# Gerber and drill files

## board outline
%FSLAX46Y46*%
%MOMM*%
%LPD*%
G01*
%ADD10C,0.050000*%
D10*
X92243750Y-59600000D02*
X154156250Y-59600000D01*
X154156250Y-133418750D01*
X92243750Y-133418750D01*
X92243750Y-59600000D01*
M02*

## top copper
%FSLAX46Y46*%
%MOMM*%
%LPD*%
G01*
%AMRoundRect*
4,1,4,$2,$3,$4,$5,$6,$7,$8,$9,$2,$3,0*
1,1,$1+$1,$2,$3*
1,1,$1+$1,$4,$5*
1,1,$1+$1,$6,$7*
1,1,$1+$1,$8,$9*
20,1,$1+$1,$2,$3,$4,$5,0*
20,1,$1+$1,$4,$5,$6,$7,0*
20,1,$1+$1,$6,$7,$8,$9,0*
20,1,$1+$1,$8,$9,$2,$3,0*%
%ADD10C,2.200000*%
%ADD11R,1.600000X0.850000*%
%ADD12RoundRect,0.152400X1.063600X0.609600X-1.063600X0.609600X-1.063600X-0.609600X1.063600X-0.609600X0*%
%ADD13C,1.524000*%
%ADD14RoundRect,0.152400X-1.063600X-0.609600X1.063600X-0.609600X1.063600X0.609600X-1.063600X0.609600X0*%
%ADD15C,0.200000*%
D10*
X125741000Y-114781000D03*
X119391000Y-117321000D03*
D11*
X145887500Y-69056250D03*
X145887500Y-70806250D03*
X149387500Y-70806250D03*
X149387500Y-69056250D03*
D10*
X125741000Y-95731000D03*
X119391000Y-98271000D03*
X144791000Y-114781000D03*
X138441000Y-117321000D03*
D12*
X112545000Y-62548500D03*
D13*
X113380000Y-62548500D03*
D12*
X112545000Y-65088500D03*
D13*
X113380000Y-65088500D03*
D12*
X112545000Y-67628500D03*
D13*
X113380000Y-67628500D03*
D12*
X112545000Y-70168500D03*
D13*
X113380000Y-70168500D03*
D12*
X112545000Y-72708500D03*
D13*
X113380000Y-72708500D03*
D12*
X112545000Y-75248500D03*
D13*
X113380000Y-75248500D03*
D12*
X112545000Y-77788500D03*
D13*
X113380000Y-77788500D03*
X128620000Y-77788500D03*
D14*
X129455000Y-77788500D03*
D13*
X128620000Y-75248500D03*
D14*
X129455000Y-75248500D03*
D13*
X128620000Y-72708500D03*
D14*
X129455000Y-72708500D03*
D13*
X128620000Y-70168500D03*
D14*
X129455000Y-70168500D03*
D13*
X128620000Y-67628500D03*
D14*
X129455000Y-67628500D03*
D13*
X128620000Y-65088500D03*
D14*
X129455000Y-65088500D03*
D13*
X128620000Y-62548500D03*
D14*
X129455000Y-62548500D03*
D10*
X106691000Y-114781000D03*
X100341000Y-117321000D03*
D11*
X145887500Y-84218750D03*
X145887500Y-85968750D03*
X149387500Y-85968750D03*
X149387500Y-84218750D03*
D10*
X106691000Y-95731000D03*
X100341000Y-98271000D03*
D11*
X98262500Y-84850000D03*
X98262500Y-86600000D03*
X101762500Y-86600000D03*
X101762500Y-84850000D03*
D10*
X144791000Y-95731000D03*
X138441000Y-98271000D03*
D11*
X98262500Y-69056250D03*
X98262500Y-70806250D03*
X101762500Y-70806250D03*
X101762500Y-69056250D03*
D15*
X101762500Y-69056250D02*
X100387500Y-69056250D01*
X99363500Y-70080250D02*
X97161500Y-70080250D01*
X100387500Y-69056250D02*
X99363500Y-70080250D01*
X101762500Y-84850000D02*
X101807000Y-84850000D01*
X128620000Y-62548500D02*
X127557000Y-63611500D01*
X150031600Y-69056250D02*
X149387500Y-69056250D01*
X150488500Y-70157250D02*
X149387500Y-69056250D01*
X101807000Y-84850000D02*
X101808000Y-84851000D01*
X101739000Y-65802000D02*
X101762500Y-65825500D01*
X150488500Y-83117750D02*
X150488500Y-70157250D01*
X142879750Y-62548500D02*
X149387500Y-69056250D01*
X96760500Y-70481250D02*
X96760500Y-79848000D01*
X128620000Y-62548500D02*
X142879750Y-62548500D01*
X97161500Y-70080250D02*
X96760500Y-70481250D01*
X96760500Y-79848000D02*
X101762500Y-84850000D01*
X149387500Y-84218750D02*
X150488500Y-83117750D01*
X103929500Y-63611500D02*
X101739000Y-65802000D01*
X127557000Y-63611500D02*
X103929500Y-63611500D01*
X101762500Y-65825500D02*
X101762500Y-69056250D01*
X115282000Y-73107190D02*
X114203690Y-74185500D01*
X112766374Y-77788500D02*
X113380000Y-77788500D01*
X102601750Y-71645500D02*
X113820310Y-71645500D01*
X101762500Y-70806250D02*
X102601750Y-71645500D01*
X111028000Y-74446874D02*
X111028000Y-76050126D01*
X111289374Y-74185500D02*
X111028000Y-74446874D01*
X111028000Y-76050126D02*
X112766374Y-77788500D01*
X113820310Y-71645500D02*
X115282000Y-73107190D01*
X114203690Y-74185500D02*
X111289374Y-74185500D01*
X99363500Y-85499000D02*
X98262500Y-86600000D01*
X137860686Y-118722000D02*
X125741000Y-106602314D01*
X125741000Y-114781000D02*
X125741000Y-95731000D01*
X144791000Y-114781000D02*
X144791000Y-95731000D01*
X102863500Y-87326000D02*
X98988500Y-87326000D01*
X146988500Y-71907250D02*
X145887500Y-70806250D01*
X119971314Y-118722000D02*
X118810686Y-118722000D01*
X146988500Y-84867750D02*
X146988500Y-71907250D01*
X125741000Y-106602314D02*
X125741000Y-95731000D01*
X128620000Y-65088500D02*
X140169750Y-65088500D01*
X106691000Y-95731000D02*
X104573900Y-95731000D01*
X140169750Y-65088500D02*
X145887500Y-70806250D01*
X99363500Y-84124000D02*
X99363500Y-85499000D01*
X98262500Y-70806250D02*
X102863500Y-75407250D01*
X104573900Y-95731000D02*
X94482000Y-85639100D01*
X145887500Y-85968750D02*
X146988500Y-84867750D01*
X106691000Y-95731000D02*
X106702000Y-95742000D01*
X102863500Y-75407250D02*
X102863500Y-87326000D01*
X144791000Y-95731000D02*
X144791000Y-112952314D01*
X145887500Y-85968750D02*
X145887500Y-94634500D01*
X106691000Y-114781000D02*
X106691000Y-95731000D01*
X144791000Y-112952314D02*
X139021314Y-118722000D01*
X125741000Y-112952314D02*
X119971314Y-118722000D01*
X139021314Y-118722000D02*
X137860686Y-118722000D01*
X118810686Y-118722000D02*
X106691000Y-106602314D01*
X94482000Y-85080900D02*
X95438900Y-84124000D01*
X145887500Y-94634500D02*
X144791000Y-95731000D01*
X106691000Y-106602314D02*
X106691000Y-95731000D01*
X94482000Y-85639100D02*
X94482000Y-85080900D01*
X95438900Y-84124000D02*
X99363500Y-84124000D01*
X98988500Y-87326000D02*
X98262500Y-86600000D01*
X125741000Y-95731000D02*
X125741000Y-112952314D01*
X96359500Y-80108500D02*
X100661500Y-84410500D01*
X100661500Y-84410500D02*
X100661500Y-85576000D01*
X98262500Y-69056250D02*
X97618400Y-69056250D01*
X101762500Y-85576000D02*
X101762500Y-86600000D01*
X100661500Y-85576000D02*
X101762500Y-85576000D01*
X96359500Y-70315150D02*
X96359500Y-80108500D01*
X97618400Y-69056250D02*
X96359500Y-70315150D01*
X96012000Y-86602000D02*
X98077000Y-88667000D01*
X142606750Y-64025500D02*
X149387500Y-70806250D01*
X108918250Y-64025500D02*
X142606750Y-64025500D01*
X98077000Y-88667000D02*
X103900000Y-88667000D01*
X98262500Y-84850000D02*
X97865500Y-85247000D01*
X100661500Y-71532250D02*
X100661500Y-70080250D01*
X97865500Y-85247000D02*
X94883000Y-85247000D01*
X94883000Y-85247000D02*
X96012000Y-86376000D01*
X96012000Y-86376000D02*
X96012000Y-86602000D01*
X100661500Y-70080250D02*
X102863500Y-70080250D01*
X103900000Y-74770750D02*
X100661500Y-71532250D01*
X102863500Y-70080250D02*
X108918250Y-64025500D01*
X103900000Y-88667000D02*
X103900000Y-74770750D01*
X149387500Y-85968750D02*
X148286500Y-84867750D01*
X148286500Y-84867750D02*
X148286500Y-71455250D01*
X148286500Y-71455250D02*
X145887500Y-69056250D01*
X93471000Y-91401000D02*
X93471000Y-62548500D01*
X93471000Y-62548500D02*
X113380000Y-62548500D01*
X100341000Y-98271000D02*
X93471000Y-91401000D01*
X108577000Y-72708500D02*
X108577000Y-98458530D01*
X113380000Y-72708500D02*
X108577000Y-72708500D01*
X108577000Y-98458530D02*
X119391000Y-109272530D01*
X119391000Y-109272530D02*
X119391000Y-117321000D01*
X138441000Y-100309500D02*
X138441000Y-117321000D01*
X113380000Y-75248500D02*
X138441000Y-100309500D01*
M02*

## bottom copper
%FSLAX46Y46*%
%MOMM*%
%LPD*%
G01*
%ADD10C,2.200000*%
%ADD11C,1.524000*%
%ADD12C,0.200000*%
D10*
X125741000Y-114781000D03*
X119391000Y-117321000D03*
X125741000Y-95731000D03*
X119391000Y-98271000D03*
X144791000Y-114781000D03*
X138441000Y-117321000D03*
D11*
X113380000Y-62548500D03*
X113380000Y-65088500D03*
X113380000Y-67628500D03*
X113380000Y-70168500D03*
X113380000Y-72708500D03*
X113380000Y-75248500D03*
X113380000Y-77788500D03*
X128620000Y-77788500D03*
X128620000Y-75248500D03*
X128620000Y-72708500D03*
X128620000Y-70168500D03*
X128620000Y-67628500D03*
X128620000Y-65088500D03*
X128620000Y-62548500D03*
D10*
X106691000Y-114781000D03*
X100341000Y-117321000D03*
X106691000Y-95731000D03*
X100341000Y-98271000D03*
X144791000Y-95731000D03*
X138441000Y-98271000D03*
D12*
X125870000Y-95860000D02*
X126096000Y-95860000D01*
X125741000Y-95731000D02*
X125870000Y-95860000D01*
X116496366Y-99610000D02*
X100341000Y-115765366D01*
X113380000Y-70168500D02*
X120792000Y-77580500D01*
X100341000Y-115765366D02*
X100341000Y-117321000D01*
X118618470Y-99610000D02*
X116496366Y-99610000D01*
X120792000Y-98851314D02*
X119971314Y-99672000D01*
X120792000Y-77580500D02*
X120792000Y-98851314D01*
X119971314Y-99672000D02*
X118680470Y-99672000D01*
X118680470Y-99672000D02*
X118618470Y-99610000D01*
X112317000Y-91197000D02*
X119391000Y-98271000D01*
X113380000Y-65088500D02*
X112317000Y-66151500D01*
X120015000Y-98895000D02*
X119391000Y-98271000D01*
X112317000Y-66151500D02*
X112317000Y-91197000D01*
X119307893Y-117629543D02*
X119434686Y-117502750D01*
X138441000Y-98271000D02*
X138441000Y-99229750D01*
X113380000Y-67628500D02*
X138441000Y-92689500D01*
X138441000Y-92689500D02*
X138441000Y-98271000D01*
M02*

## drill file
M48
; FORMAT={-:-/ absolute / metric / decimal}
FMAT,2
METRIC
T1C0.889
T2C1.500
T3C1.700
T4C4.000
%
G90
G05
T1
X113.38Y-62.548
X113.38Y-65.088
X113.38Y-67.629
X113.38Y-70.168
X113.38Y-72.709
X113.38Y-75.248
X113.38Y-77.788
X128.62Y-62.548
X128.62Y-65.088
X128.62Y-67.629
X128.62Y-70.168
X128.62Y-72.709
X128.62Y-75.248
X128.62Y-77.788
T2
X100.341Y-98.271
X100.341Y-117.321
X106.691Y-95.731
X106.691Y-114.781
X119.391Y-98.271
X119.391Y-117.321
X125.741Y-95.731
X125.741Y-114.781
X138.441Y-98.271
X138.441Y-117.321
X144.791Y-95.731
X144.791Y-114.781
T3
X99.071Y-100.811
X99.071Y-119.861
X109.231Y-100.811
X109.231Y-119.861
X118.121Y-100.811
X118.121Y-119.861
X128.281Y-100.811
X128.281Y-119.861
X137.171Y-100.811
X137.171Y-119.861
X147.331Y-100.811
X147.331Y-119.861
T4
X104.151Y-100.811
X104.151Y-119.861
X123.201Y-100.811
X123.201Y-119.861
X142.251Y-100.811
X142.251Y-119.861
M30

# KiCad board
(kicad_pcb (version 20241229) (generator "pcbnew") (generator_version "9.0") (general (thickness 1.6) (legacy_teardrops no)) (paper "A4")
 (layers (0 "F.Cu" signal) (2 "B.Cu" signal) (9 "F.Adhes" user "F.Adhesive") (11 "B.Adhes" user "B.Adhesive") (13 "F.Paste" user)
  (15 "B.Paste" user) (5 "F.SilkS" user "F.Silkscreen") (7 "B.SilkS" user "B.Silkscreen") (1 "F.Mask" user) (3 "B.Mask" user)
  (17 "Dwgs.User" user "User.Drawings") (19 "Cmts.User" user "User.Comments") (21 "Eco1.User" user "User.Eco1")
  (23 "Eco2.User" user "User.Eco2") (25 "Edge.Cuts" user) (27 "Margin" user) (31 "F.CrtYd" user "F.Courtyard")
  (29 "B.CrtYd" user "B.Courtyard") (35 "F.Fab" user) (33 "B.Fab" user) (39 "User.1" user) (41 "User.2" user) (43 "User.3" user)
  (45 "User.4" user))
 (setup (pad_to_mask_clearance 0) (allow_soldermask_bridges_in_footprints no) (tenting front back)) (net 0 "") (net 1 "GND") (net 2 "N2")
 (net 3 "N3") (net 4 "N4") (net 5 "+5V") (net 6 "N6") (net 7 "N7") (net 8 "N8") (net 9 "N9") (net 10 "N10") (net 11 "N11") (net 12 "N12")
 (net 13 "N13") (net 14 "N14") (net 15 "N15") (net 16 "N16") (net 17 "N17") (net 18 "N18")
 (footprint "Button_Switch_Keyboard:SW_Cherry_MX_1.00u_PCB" (layer "F.Cu") (at 125.741 114.781)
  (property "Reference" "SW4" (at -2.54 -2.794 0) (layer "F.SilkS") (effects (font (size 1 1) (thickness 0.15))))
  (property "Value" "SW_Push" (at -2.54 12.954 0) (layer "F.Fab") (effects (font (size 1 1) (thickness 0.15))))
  (pad "" np_thru_hole circle (at -7.62 5.08) (size 1.7 1.7) (drill 1.7) (layers "*.Cu" "*.Mask"))
  (pad "" np_thru_hole circle (at -2.54 5.08) (size 4 4) (drill 4) (layers "*.Cu" "*.Mask"))
  (pad "" np_thru_hole circle (at 2.54 5.08) (size 1.7 1.7) (drill 1.7) (layers "*.Cu" "*.Mask"))
  (pad "1" thru_hole circle (at 0 0) (size 2.2 2.2) (drill 1.5) (layers "*.Cu" "*.Mask") (remove_unused_layers no) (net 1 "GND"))
  (pad "2" thru_hole circle (at -6.35 2.54) (size 2.2 2.2) (drill 1.5) (layers "*.Cu" "*.Mask") (remove_unused_layers no) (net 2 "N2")))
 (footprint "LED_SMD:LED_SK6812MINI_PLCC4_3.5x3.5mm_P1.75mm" (layer "F.Cu") (at 147.6375 69.93125)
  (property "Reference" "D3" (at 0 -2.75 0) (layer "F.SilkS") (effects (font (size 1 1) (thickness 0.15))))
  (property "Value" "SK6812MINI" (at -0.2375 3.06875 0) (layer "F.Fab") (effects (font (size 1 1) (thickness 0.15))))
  (pad "1" smd rect (at -1.75 -0.875) (size 1.6 0.85) (layers "F.Cu" "F.Mask" "F.Paste") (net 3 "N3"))
  (pad "2" smd rect (at -1.75 0.875) (size 1.6 0.85) (layers "F.Cu" "F.Mask" "F.Paste") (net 1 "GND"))
  (pad "3" smd rect (at 1.75 0.875) (size 1.6 0.85) (layers "F.Cu" "F.Mask" "F.Paste") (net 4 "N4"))
  (pad "4" smd rect (at 1.75 -0.875) (size 1.6 0.85) (layers "F.Cu" "F.Mask" "F.Paste") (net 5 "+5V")))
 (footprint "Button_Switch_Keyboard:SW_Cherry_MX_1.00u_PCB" (layer "F.Cu") (at 125.741 95.731)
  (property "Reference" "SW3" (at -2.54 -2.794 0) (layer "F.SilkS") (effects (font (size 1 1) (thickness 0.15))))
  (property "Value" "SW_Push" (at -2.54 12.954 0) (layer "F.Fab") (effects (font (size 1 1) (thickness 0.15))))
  (pad "" np_thru_hole circle (at -7.62 5.08) (size 1.7 1.7) (drill 1.7) (layers "*.Cu" "*.Mask"))
  (pad "" np_thru_hole circle (at -2.54 5.08) (size 4 4) (drill 4) (layers "*.Cu" "*.Mask"))
  (pad "" np_thru_hole circle (at 2.54 5.08) (size 1.7 1.7) (drill 1.7) (layers "*.Cu" "*.Mask"))
  (pad "1" thru_hole circle (at 0 0) (size 2.2 2.2) (drill 1.5) (layers "*.Cu" "*.Mask") (remove_unused_layers no) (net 1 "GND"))
  (pad "2" thru_hole circle (at -6.35 2.54) (size 2.2 2.2) (drill 1.5) (layers "*.Cu" "*.Mask") (remove_unused_layers no) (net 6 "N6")))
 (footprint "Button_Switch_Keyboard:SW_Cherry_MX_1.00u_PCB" (layer "F.Cu") (at 144.791 114.781)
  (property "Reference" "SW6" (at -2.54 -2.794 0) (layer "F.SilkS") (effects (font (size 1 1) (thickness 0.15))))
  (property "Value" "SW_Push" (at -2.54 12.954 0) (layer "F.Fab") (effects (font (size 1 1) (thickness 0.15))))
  (pad "" np_thru_hole circle (at -7.62 5.08) (size 1.7 1.7) (drill 1.7) (layers "*.Cu" "*.Mask"))
  (pad "" np_thru_hole circle (at -2.54 5.08) (size 4 4) (drill 4) (layers "*.Cu" "*.Mask"))
  (pad "" np_thru_hole circle (at 2.54 5.08) (size 1.7 1.7) (drill 1.7) (layers "*.Cu" "*.Mask"))
  (pad "1" thru_hole circle (at 0 0) (size 2.2 2.2) (drill 1.5) (layers "*.Cu" "*.Mask") (remove_unused_layers no) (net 1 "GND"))
  (pad "2" thru_hole circle (at -6.35 2.54) (size 2.2 2.2) (drill 1.5) (layers "*.Cu" "*.Mask") (remove_unused_layers no) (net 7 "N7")))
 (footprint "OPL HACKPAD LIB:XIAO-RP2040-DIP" (layer "F.Cu") (at 121 70.1685)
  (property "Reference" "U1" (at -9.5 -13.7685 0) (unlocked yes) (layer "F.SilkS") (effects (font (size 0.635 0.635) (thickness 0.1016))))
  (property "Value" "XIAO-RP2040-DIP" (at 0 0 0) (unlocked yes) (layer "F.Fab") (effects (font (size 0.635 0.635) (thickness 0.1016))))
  (pad "1" smd roundrect (at -8.455 -7.62 180) (size 2.432 1.524) (layers "F.Cu" "F.Mask") (roundrect_rratio 0.1) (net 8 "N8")
   (thermal_bridge_angle 45))
  (pad "1" thru_hole circle (at -7.62 -7.62 180) (size 1.524 1.524) (drill 0.889) (layers "*.Cu" "*.Mask") (remove_unused_layers no)
   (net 8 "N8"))
  (pad "2" smd roundrect (at -8.455 -5.08 180) (size 2.432 1.524) (layers "F.Cu" "F.Mask") (roundrect_rratio 0.1) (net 6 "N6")
   (thermal_bridge_angle 45))
  (pad "2" thru_hole circle (at -7.62 -5.08 180) (size 1.524 1.524) (drill 0.889) (layers "*.Cu" "*.Mask") (remove_unused_layers no)
   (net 6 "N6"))
  (pad "3" smd roundrect (at -8.455 -2.54 180) (size 2.432 1.524) (layers "F.Cu" "F.Mask") (roundrect_rratio 0.1) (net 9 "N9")
   (thermal_bridge_angle 45))
  (pad "3" thru_hole circle (at -7.62 -2.54 180) (size 1.524 1.524) (drill 0.889) (layers "*.Cu" "*.Mask") (remove_unused_layers no)
   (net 9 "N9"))
  (pad "4" smd roundrect (at -8.455 0 180) (size 2.432 1.524) (layers "F.Cu" "F.Mask") (roundrect_rratio 0.1) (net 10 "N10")
   (thermal_bridge_angle 45))
  (pad "4" thru_hole circle (at -7.62 0 180) (size 1.524 1.524) (drill 0.889) (layers "*.Cu" "*.Mask") (remove_unused_layers no)
   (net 10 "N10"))
  (pad "5" smd roundrect (at -8.455 2.54 180) (size 2.432 1.524) (layers "F.Cu" "F.Mask") (roundrect_rratio 0.1) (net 2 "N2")
   (thermal_bridge_angle 45))
  (pad "5" thru_hole circle (at -7.62 2.54 180) (size 1.524 1.524) (drill 0.889) (layers "*.Cu" "*.Mask") (remove_unused_layers no)
   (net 2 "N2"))
  (pad "6" smd roundrect (at -8.455 5.08 180) (size 2.432 1.524) (layers "F.Cu" "F.Mask") (roundrect_rratio 0.1) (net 7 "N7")
   (thermal_bridge_angle 45))
  (pad "6" thru_hole circle (at -7.62 5.08 180) (size 1.524 1.524) (drill 0.889) (layers "*.Cu" "*.Mask") (remove_unused_layers no)
   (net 7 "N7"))
  (pad "7" smd roundrect (at -8.455 7.62 180) (size 2.432 1.524) (layers "F.Cu" "F.Mask") (roundrect_rratio 0.1) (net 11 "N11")
   (thermal_bridge_angle 45))
  (pad "7" thru_hole circle (at -7.62 7.62 180) (size 1.524 1.524) (drill 0.889) (layers "*.Cu" "*.Mask") (remove_unused_layers no)
   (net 11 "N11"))
  (pad "8" thru_hole circle (at 7.62 7.62) (size 1.524 1.524) (drill 0.889) (layers "*.Cu" "*.Mask") (remove_unused_layers no)
   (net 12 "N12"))
  (pad "8" smd roundrect (at 8.455 7.62) (size 2.432 1.524) (layers "F.Cu" "F.Mask") (roundrect_rratio 0.1) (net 12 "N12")
   (thermal_bridge_angle 45))
  (pad "9" thru_hole circle (at 7.62 5.08) (size 1.524 1.524) (drill 0.889) (layers "*.Cu" "*.Mask") (remove_unused_layers no)
   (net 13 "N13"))
  (pad "9" smd roundrect (at 8.455 5.08) (size 2.432 1.524) (layers "F.Cu" "F.Mask") (roundrect_rratio 0.1) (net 13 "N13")
   (thermal_bridge_angle 45))
  (pad "10" thru_hole circle (at 7.62 2.54) (size 1.524 1.524) (drill 0.889) (layers "*.Cu" "*.Mask") (remove_unused_layers no)
   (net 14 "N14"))
  (pad "10" smd roundrect (at 8.455 2.54) (size 2.432 1.524) (layers "F.Cu" "F.Mask") (roundrect_rratio 0.1) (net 14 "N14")
   (thermal_bridge_angle 45))
  (pad "11" thru_hole circle (at 7.62 0) (size 1.524 1.524) (drill 0.889) (layers "*.Cu" "*.Mask") (remove_unused_layers no) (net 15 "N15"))
  (pad "11" smd roundrect (at 8.455 0) (size 2.432 1.524) (layers "F.Cu" "F.Mask") (roundrect_rratio 0.1) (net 15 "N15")
   (thermal_bridge_angle 45))
  (pad "12" thru_hole circle (at 7.62 -2.54) (size 1.524 1.524) (drill 0.889) (layers "*.Cu" "*.Mask") (remove_unused_layers no)
   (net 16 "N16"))
  (pad "12" smd roundrect (at 8.455 -2.54) (size 2.432 1.524) (layers "F.Cu" "F.Mask") (roundrect_rratio 0.1) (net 16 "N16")
   (thermal_bridge_angle 45))
  (pad "13" thru_hole circle (at 7.62 -5.08) (size 1.524 1.524) (drill 0.889) (layers "*.Cu" "*.Mask") (remove_unused_layers no)
   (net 1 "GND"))
  (pad "13" smd roundrect (at 8.455 -5.08) (size 2.432 1.524) (layers "F.Cu" "F.Mask") (roundrect_rratio 0.1) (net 1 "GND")
   (thermal_bridge_angle 45))
  (pad "14" thru_hole circle (at 7.62 -7.62) (size 1.524 1.524) (drill 0.889) (layers "*.Cu" "*.Mask") (remove_unused_layers no)
   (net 5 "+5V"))
  (pad "14" smd roundrect (at 8.455 -7.62) (size 2.432 1.524) (layers "F.Cu" "F.Mask") (roundrect_rratio 0.1) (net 5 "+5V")
   (thermal_bridge_angle 45)))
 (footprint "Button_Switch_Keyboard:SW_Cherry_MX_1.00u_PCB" (layer "F.Cu") (at 106.691 114.781)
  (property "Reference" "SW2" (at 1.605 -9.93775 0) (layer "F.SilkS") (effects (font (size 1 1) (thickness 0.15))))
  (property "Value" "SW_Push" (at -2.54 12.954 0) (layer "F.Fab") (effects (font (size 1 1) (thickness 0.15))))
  (pad "" np_thru_hole circle (at -7.62 5.08) (size 1.7 1.7) (drill 1.7) (layers "*.Cu" "*.Mask"))
  (pad "" np_thru_hole circle (at -2.54 5.08) (size 4 4) (drill 4) (layers "*.Cu" "*.Mask"))
  (pad "" np_thru_hole circle (at 2.54 5.08) (size 1.7 1.7) (drill 1.7) (layers "*.Cu" "*.Mask"))
  (pad "1" thru_hole circle (at 0 0) (size 2.2 2.2) (drill 1.5) (layers "*.Cu" "*.Mask") (remove_unused_layers no) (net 1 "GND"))
  (pad "2" thru_hole circle (at -6.35 2.54) (size 2.2 2.2) (drill 1.5) (layers "*.Cu" "*.Mask") (remove_unused_layers no) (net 10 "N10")))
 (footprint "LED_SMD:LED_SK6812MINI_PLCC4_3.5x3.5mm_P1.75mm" (layer "F.Cu") (at 147.6375 85.09375)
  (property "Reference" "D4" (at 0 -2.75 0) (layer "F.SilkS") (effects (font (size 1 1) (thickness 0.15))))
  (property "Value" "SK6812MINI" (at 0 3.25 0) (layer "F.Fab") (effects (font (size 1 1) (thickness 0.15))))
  (pad "1" smd rect (at -1.75 -0.875) (size 1.6 0.85) (layers "F.Cu" "F.Mask" "F.Paste") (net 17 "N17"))
  (pad "2" smd rect (at -1.75 0.875) (size 1.6 0.85) (layers "F.Cu" "F.Mask" "F.Paste") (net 1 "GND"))
  (pad "3" smd rect (at 1.75 0.875) (size 1.6 0.85) (layers "F.Cu" "F.Mask" "F.Paste") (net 3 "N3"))
  (pad "4" smd rect (at 1.75 -0.875) (size 1.6 0.85) (layers "F.Cu" "F.Mask" "F.Paste") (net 5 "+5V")))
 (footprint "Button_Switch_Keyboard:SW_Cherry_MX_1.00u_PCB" (layer "F.Cu") (at 106.691 95.731)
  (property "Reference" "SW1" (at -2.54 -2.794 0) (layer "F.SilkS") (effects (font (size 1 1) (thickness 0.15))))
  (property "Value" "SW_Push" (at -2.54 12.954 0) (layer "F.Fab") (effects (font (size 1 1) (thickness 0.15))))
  (pad "" np_thru_hole circle (at -7.62 5.08) (size 1.7 1.7) (drill 1.7) (layers "*.Cu" "*.Mask"))
  (pad "" np_thru_hole circle (at -2.54 5.08) (size 4 4) (drill 4) (layers "*.Cu" "*.Mask"))
  (pad "" np_thru_hole circle (at 2.54 5.08) (size 1.7 1.7) (drill 1.7) (layers "*.Cu" "*.Mask"))
  (pad "1" thru_hole circle (at 0 0) (size 2.2 2.2) (drill 1.5) (layers "*.Cu" "*.Mask") (remove_unused_layers no) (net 1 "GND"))
  (pad "2" thru_hole circle (at -6.35 2.54) (size 2.2 2.2) (drill 1.5) (layers "*.Cu" "*.Mask") (remove_unused_layers no) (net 8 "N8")))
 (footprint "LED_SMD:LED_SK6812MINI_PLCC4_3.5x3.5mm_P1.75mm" (layer "F.Cu") (at 100.0125 85.725)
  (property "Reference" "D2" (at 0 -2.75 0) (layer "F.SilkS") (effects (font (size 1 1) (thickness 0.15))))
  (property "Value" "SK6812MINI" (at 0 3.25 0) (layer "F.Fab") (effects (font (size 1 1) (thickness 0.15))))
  (pad "1" smd rect (at -1.75 -0.875) (size 1.6 0.85) (layers "F.Cu" "F.Mask" "F.Paste") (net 4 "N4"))
  (pad "2" smd rect (at -1.75 0.875) (size 1.6 0.85) (layers "F.Cu" "F.Mask" "F.Paste") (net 1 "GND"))
  (pad "3" smd rect (at 1.75 0.875) (size 1.6 0.85) (layers "F.Cu" "F.Mask" "F.Paste") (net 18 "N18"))
  (pad "4" smd rect (at 1.75 -0.875) (size 1.6 0.85) (layers "F.Cu" "F.Mask" "F.Paste") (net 5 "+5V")))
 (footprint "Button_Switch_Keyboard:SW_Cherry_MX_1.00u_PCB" (layer "F.Cu") (at 144.791 95.731)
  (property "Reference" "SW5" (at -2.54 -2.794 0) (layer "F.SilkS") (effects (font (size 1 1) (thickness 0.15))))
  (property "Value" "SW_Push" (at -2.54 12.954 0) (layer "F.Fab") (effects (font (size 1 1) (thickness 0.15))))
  (pad "" np_thru_hole circle (at -7.62 5.08) (size 1.7 1.7) (drill 1.7) (layers "*.Cu" "*.Mask"))
  (pad "" np_thru_hole circle (at -2.54 5.08) (size 4 4) (drill 4) (layers "*.Cu" "*.Mask"))
  (pad "" np_thru_hole circle (at 2.54 5.08) (size 1.7 1.7) (drill 1.7) (layers "*.Cu" "*.Mask"))
  (pad "1" thru_hole circle (at 0 0) (size 2.2 2.2) (drill 1.5) (layers "*.Cu" "*.Mask") (remove_unused_layers no) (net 1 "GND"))
  (pad "2" thru_hole circle (at -6.35 2.54) (size 2.2 2.2) (drill 1.5) (layers "*.Cu" "*.Mask") (remove_unused_layers no) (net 9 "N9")))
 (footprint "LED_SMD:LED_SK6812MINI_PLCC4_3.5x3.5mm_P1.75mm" (layer "F.Cu") (at 100.0125 69.93125)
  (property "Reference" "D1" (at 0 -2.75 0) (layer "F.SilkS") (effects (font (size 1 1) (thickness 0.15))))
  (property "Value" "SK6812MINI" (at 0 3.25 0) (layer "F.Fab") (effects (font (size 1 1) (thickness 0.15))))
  (pad "1" smd rect (at -1.75 -0.875) (size 1.6 0.85) (layers "F.Cu" "F.Mask" "F.Paste") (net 18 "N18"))
  (pad "2" smd rect (at -1.75 0.875) (size 1.6 0.85) (layers "F.Cu" "F.Mask" "F.Paste") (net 1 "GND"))
  (pad "3" smd rect (at 1.75 0.875) (size 1.6 0.85) (layers "F.Cu" "F.Mask" "F.Paste") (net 11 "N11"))
  (pad "4" smd rect (at 1.75 -0.875) (size 1.6 0.85) (layers "F.Cu" "F.Mask" "F.Paste") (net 5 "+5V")))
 (gr_rect (start 92.24375 59.6) (end 154.15625 133.41875) (stroke (width 0.05) (type default)) (fill no) (layer "Edge.Cuts"))
 (segment (start 101.7625 69.05625) (end 100.3875 69.05625) (width 0.2) (layer "F.Cu") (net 5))
 (segment (start 99.3635 70.08025) (end 97.1615 70.08025) (width 0.2) (layer "F.Cu") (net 5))
 (segment (start 100.3875 69.05625) (end 99.3635 70.08025) (width 0.2) (layer "F.Cu") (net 5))
 (segment (start 101.7625 84.85) (end 101.807 84.85) (width 0.2) (layer "F.Cu") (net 5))
 (segment (start 128.62 62.5485) (end 127.557 63.6115) (width 0.2) (layer "F.Cu") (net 5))
 (segment (start 150.0316 69.05625) (end 149.3875 69.05625) (width 0.2) (layer "F.Cu") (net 5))
 (segment (start 150.4885 70.15725) (end 149.3875 69.05625) (width 0.2) (layer "F.Cu") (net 5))
 (segment (start 101.807 84.85) (end 101.808 84.851) (width 0.2) (layer "F.Cu") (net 5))
 (segment (start 101.739 65.802) (end 101.7625 65.8255) (width 0.2) (layer "F.Cu") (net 5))
 (segment (start 150.4885 83.11775) (end 150.4885 70.15725) (width 0.2) (layer "F.Cu") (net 5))
 (segment (start 142.87975 62.5485) (end 149.3875 69.05625) (width 0.2) (layer "F.Cu") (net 5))
 (segment (start 96.7605 70.48125) (end 96.7605 79.848) (width 0.2) (layer "F.Cu") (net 5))
 (segment (start 128.62 62.5485) (end 142.87975 62.5485) (width 0.2) (layer "F.Cu") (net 5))
 (segment (start 97.1615 70.08025) (end 96.7605 70.48125) (width 0.2) (layer "F.Cu") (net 5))
 (segment (start 96.7605 79.848) (end 101.7625 84.85) (width 0.2) (layer "F.Cu") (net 5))
 (segment (start 149.3875 84.21875) (end 150.4885 83.11775) (width 0.2) (layer "F.Cu") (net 5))
 (segment (start 103.9295 63.6115) (end 101.739 65.802) (width 0.2) (layer "F.Cu") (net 5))
 (segment (start 127.557 63.6115) (end 103.9295 63.6115) (width 0.2) (layer "F.Cu") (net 5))
 (segment (start 101.7625 65.8255) (end 101.7625 69.05625) (width 0.2) (layer "F.Cu") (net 5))
 (segment (start 115.282 73.10719) (end 114.20369 74.1855) (width 0.2) (layer "F.Cu") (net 11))
 (segment (start 112.766374 77.7885) (end 113.38 77.7885) (width 0.2) (layer "F.Cu") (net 11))
 (segment (start 102.60175 71.6455) (end 113.82031 71.6455) (width 0.2) (layer "F.Cu") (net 11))
 (segment (start 101.7625 70.80625) (end 102.60175 71.6455) (width 0.2) (layer "F.Cu") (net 11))
 (segment (start 111.028 74.446874) (end 111.028 76.050126) (width 0.2) (layer "F.Cu") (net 11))
 (segment (start 111.289374 74.1855) (end 111.028 74.446874) (width 0.2) (layer "F.Cu") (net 11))
 (segment (start 111.028 76.050126) (end 112.766374 77.7885) (width 0.2) (layer "F.Cu") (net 11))
 (segment (start 113.82031 71.6455) (end 115.282 73.10719) (width 0.2) (layer "F.Cu") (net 11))
 (segment (start 114.20369 74.1855) (end 111.289374 74.1855) (width 0.2) (layer "F.Cu") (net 11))
 (segment (start 99.3635 85.499) (end 98.2625 86.6) (width 0.2) (layer "F.Cu") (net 1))
 (segment (start 137.860686 118.722) (end 125.741 106.602314) (width 0.2) (layer "F.Cu") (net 1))
 (segment (start 125.741 114.781) (end 125.741 95.731) (width 0.2) (layer "F.Cu") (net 1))
 (segment (start 144.791 114.781) (end 144.791 95.731) (width 0.2) (layer "F.Cu") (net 1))
 (segment (start 102.8635 87.326) (end 98.9885 87.326) (width 0.2) (layer "F.Cu") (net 1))
 (segment (start 146.9885 71.90725) (end 145.8875 70.80625) (width 0.2) (layer "F.Cu") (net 1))
 (segment (start 119.971314 118.722) (end 118.810686 118.722) (width 0.2) (layer "F.Cu") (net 1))
 (segment (start 146.9885 84.86775) (end 146.9885 71.90725) (width 0.2) (layer "F.Cu") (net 1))
 (segment (start 125.741 106.602314) (end 125.741 95.731) (width 0.2) (layer "F.Cu") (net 1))
 (segment (start 128.62 65.0885) (end 140.16975 65.0885) (width 0.2) (layer "F.Cu") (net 1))
 (segment (start 106.691 95.731) (end 104.5739 95.731) (width 0.2) (layer "F.Cu") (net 1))
 (segment (start 140.16975 65.0885) (end 145.8875 70.80625) (width 0.2) (layer "F.Cu") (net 1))
 (segment (start 99.3635 84.124) (end 99.3635 85.499) (width 0.2) (layer "F.Cu") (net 1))
 (segment (start 98.2625 70.80625) (end 102.8635 75.40725) (width 0.2) (layer "F.Cu") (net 1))
 (segment (start 104.5739 95.731) (end 94.482 85.6391) (width 0.2) (layer "F.Cu") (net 1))
 (segment (start 145.8875 85.96875) (end 146.9885 84.86775) (width 0.2) (layer "F.Cu") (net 1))
 (segment (start 106.691 95.731) (end 106.702 95.742) (width 0.2) (layer "F.Cu") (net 1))
 (segment (start 102.8635 75.40725) (end 102.8635 87.326) (width 0.2) (layer "F.Cu") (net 1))
 (segment (start 144.791 95.731) (end 144.791 112.952314) (width 0.2) (layer "F.Cu") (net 1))
 (segment (start 145.8875 85.96875) (end 145.8875 94.6345) (width 0.2) (layer "F.Cu") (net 1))
 (segment (start 106.691 114.781) (end 106.691 95.731) (width 0.2) (layer "F.Cu") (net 1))
 (segment (start 144.791 112.952314) (end 139.021314 118.722) (width 0.2) (layer "F.Cu") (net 1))
 (segment (start 125.741 112.952314) (end 119.971314 118.722) (width 0.2) (layer "F.Cu") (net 1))
 (segment (start 139.021314 118.722) (end 137.860686 118.722) (width 0.2) (layer "F.Cu") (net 1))
 (segment (start 118.810686 118.722) (end 106.691 106.602314) (width 0.2) (layer "F.Cu") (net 1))
 (segment (start 94.482 85.0809) (end 95.4389 84.124) (width 0.2) (layer "F.Cu") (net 1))
 (segment (start 145.8875 94.6345) (end 144.791 95.731) (width 0.2) (layer "F.Cu") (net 1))
 (segment (start 106.691 106.602314) (end 106.691 95.731) (width 0.2) (layer "F.Cu") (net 1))
 (segment (start 94.482 85.6391) (end 94.482 85.0809) (width 0.2) (layer "F.Cu") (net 1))
 (segment (start 95.4389 84.124) (end 99.3635 84.124) (width 0.2) (layer "F.Cu") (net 1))
 (segment (start 98.9885 87.326) (end 98.2625 86.6) (width 0.2) (layer "F.Cu") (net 1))
 (segment (start 125.741 95.731) (end 125.741 112.952314) (width 0.2) (layer "F.Cu") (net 1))
 (segment (start 125.87 95.86) (end 126.096 95.86) (width 0.2) (layer "B.Cu") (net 1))
 (segment (start 125.741 95.731) (end 125.87 95.86) (width 0.2) (layer "B.Cu") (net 1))
 (segment (start 96.3595 80.1085) (end 100.6615 84.4105) (width 0.2) (layer "F.Cu") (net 18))
 (segment (start 100.6615 84.4105) (end 100.6615 85.576) (width 0.2) (layer "F.Cu") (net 18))
 (segment (start 98.2625 69.05625) (end 97.6184 69.05625) (width 0.2) (layer "F.Cu") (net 18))
 (segment (start 101.7625 85.576) (end 101.7625 86.6) (width 0.2) (layer "F.Cu") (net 18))
 (segment (start 100.6615 85.576) (end 101.7625 85.576) (width 0.2) (layer "F.Cu") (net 18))
 (segment (start 96.3595 70.31515) (end 96.3595 80.1085) (width 0.2) (layer "F.Cu") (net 18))
 (segment (start 97.6184 69.05625) (end 96.3595 70.31515) (width 0.2) (layer "F.Cu") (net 18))
 (segment (start 96.012 86.602) (end 98.077 88.667) (width 0.2) (layer "F.Cu") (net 4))
 (segment (start 142.60675 64.0255) (end 149.3875 70.80625) (width 0.2) (layer "F.Cu") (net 4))
 (segment (start 108.91825 64.0255) (end 142.60675 64.0255) (width 0.2) (layer "F.Cu") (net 4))
 (segment (start 98.077 88.667) (end 103.9 88.667) (width 0.2) (layer "F.Cu") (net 4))
 (segment (start 98.2625 84.85) (end 97.8655 85.247) (width 0.2) (layer "F.Cu") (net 4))
 (segment (start 100.6615 71.53225) (end 100.6615 70.08025) (width 0.2) (layer "F.Cu") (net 4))
 (segment (start 97.8655 85.247) (end 94.883 85.247) (width 0.2) (layer "F.Cu") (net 4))
 (segment (start 94.883 85.247) (end 96.012 86.376) (width 0.2) (layer "F.Cu") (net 4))
 (segment (start 96.012 86.376) (end 96.012 86.602) (width 0.2) (layer "F.Cu") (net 4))
 (segment (start 100.6615 70.08025) (end 102.8635 70.08025) (width 0.2) (layer "F.Cu") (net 4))
 (segment (start 103.9 74.77075) (end 100.6615 71.53225) (width 0.2) (layer "F.Cu") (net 4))
 (segment (start 102.8635 70.08025) (end 108.91825 64.0255) (width 0.2) (layer "F.Cu") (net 4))
 (segment (start 103.9 88.667) (end 103.9 74.77075) (width 0.2) (layer "F.Cu") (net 4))
 (segment (start 149.3875 85.96875) (end 148.2865 84.86775) (width 0.2) (layer "F.Cu") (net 3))
 (segment (start 148.2865 84.86775) (end 148.2865 71.45525) (width 0.2) (layer "F.Cu") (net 3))
 (segment (start 148.2865 71.45525) (end 145.8875 69.05625) (width 0.2) (layer "F.Cu") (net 3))
 (segment (start 93.471 91.401) (end 93.471 62.5485) (width 0.2) (layer "F.Cu") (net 8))
 (segment (start 93.471 62.5485) (end 113.38 62.5485) (width 0.2) (layer "F.Cu") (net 8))
 (segment (start 100.341 98.271) (end 93.471 91.401) (width 0.2) (layer "F.Cu") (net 8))
 (segment (start 116.496366 99.61) (end 100.341 115.765366) (width 0.2) (layer "B.Cu") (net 10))
 (segment (start 113.38 70.1685) (end 120.792 77.5805) (width 0.2) (layer "B.Cu") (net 10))
 (segment (start 100.341 115.765366) (end 100.341 117.321) (width 0.2) (layer "B.Cu") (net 10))
 (segment (start 118.61847 99.61) (end 116.496366 99.61) (width 0.2) (layer "B.Cu") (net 10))
 (segment (start 120.792 98.851314) (end 119.971314 99.672) (width 0.2) (layer "B.Cu") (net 10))
 (segment (start 120.792 77.5805) (end 120.792 98.851314) (width 0.2) (layer "B.Cu") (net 10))
 (segment (start 119.971314 99.672) (end 118.68047 99.672) (width 0.2) (layer "B.Cu") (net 10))
 (segment (start 118.68047 99.672) (end 118.61847 99.61) (width 0.2) (layer "B.Cu") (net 10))
 (segment (start 112.317 91.197) (end 119.391 98.271) (width 0.2) (layer "B.Cu") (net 6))
 (segment (start 113.38 65.0885) (end 112.317 66.1515) (width 0.2) (layer "B.Cu") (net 6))
 (segment (start 120.015 98.895) (end 119.391 98.271) (width 0.2) (layer "B.Cu") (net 6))
 (segment (start 112.317 66.1515) (end 112.317 91.197) (width 0.2) (layer "B.Cu") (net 6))
 (segment (start 108.577 72.7085) (end 108.577 98.45853) (width 0.2) (layer "F.Cu") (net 2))
 (segment (start 113.38 72.7085) (end 108.577 72.7085) (width 0.2) (layer "F.Cu") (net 2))
 (segment (start 108.577 98.45853) (end 119.391 109.27253) (width 0.2) (layer "F.Cu") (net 2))
 (segment (start 119.391 109.27253) (end 119.391 117.321) (width 0.2) (layer "F.Cu") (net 2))
 (segment (start 119.307893 117.629543) (end 119.434686 117.50275) (width 0.2) (layer "B.Cu") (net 2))
 (segment (start 138.441 98.271) (end 138.441 99.22975) (width 0.2) (layer "B.Cu") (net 9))
 (segment (start 113.38 67.6285) (end 138.441 92.6895) (width 0.2) (layer "B.Cu") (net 9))
 (segment (start 138.441 92.6895) (end 138.441 98.271) (width 0.2) (layer "B.Cu") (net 9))
 (segment (start 138.441 100.3095) (end 138.441 117.321) (width 0.2) (layer "F.Cu") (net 7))
 (segment (start 113.38 75.2485) (end 138.441 100.3095) (width 0.2) (layer "F.Cu") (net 7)))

